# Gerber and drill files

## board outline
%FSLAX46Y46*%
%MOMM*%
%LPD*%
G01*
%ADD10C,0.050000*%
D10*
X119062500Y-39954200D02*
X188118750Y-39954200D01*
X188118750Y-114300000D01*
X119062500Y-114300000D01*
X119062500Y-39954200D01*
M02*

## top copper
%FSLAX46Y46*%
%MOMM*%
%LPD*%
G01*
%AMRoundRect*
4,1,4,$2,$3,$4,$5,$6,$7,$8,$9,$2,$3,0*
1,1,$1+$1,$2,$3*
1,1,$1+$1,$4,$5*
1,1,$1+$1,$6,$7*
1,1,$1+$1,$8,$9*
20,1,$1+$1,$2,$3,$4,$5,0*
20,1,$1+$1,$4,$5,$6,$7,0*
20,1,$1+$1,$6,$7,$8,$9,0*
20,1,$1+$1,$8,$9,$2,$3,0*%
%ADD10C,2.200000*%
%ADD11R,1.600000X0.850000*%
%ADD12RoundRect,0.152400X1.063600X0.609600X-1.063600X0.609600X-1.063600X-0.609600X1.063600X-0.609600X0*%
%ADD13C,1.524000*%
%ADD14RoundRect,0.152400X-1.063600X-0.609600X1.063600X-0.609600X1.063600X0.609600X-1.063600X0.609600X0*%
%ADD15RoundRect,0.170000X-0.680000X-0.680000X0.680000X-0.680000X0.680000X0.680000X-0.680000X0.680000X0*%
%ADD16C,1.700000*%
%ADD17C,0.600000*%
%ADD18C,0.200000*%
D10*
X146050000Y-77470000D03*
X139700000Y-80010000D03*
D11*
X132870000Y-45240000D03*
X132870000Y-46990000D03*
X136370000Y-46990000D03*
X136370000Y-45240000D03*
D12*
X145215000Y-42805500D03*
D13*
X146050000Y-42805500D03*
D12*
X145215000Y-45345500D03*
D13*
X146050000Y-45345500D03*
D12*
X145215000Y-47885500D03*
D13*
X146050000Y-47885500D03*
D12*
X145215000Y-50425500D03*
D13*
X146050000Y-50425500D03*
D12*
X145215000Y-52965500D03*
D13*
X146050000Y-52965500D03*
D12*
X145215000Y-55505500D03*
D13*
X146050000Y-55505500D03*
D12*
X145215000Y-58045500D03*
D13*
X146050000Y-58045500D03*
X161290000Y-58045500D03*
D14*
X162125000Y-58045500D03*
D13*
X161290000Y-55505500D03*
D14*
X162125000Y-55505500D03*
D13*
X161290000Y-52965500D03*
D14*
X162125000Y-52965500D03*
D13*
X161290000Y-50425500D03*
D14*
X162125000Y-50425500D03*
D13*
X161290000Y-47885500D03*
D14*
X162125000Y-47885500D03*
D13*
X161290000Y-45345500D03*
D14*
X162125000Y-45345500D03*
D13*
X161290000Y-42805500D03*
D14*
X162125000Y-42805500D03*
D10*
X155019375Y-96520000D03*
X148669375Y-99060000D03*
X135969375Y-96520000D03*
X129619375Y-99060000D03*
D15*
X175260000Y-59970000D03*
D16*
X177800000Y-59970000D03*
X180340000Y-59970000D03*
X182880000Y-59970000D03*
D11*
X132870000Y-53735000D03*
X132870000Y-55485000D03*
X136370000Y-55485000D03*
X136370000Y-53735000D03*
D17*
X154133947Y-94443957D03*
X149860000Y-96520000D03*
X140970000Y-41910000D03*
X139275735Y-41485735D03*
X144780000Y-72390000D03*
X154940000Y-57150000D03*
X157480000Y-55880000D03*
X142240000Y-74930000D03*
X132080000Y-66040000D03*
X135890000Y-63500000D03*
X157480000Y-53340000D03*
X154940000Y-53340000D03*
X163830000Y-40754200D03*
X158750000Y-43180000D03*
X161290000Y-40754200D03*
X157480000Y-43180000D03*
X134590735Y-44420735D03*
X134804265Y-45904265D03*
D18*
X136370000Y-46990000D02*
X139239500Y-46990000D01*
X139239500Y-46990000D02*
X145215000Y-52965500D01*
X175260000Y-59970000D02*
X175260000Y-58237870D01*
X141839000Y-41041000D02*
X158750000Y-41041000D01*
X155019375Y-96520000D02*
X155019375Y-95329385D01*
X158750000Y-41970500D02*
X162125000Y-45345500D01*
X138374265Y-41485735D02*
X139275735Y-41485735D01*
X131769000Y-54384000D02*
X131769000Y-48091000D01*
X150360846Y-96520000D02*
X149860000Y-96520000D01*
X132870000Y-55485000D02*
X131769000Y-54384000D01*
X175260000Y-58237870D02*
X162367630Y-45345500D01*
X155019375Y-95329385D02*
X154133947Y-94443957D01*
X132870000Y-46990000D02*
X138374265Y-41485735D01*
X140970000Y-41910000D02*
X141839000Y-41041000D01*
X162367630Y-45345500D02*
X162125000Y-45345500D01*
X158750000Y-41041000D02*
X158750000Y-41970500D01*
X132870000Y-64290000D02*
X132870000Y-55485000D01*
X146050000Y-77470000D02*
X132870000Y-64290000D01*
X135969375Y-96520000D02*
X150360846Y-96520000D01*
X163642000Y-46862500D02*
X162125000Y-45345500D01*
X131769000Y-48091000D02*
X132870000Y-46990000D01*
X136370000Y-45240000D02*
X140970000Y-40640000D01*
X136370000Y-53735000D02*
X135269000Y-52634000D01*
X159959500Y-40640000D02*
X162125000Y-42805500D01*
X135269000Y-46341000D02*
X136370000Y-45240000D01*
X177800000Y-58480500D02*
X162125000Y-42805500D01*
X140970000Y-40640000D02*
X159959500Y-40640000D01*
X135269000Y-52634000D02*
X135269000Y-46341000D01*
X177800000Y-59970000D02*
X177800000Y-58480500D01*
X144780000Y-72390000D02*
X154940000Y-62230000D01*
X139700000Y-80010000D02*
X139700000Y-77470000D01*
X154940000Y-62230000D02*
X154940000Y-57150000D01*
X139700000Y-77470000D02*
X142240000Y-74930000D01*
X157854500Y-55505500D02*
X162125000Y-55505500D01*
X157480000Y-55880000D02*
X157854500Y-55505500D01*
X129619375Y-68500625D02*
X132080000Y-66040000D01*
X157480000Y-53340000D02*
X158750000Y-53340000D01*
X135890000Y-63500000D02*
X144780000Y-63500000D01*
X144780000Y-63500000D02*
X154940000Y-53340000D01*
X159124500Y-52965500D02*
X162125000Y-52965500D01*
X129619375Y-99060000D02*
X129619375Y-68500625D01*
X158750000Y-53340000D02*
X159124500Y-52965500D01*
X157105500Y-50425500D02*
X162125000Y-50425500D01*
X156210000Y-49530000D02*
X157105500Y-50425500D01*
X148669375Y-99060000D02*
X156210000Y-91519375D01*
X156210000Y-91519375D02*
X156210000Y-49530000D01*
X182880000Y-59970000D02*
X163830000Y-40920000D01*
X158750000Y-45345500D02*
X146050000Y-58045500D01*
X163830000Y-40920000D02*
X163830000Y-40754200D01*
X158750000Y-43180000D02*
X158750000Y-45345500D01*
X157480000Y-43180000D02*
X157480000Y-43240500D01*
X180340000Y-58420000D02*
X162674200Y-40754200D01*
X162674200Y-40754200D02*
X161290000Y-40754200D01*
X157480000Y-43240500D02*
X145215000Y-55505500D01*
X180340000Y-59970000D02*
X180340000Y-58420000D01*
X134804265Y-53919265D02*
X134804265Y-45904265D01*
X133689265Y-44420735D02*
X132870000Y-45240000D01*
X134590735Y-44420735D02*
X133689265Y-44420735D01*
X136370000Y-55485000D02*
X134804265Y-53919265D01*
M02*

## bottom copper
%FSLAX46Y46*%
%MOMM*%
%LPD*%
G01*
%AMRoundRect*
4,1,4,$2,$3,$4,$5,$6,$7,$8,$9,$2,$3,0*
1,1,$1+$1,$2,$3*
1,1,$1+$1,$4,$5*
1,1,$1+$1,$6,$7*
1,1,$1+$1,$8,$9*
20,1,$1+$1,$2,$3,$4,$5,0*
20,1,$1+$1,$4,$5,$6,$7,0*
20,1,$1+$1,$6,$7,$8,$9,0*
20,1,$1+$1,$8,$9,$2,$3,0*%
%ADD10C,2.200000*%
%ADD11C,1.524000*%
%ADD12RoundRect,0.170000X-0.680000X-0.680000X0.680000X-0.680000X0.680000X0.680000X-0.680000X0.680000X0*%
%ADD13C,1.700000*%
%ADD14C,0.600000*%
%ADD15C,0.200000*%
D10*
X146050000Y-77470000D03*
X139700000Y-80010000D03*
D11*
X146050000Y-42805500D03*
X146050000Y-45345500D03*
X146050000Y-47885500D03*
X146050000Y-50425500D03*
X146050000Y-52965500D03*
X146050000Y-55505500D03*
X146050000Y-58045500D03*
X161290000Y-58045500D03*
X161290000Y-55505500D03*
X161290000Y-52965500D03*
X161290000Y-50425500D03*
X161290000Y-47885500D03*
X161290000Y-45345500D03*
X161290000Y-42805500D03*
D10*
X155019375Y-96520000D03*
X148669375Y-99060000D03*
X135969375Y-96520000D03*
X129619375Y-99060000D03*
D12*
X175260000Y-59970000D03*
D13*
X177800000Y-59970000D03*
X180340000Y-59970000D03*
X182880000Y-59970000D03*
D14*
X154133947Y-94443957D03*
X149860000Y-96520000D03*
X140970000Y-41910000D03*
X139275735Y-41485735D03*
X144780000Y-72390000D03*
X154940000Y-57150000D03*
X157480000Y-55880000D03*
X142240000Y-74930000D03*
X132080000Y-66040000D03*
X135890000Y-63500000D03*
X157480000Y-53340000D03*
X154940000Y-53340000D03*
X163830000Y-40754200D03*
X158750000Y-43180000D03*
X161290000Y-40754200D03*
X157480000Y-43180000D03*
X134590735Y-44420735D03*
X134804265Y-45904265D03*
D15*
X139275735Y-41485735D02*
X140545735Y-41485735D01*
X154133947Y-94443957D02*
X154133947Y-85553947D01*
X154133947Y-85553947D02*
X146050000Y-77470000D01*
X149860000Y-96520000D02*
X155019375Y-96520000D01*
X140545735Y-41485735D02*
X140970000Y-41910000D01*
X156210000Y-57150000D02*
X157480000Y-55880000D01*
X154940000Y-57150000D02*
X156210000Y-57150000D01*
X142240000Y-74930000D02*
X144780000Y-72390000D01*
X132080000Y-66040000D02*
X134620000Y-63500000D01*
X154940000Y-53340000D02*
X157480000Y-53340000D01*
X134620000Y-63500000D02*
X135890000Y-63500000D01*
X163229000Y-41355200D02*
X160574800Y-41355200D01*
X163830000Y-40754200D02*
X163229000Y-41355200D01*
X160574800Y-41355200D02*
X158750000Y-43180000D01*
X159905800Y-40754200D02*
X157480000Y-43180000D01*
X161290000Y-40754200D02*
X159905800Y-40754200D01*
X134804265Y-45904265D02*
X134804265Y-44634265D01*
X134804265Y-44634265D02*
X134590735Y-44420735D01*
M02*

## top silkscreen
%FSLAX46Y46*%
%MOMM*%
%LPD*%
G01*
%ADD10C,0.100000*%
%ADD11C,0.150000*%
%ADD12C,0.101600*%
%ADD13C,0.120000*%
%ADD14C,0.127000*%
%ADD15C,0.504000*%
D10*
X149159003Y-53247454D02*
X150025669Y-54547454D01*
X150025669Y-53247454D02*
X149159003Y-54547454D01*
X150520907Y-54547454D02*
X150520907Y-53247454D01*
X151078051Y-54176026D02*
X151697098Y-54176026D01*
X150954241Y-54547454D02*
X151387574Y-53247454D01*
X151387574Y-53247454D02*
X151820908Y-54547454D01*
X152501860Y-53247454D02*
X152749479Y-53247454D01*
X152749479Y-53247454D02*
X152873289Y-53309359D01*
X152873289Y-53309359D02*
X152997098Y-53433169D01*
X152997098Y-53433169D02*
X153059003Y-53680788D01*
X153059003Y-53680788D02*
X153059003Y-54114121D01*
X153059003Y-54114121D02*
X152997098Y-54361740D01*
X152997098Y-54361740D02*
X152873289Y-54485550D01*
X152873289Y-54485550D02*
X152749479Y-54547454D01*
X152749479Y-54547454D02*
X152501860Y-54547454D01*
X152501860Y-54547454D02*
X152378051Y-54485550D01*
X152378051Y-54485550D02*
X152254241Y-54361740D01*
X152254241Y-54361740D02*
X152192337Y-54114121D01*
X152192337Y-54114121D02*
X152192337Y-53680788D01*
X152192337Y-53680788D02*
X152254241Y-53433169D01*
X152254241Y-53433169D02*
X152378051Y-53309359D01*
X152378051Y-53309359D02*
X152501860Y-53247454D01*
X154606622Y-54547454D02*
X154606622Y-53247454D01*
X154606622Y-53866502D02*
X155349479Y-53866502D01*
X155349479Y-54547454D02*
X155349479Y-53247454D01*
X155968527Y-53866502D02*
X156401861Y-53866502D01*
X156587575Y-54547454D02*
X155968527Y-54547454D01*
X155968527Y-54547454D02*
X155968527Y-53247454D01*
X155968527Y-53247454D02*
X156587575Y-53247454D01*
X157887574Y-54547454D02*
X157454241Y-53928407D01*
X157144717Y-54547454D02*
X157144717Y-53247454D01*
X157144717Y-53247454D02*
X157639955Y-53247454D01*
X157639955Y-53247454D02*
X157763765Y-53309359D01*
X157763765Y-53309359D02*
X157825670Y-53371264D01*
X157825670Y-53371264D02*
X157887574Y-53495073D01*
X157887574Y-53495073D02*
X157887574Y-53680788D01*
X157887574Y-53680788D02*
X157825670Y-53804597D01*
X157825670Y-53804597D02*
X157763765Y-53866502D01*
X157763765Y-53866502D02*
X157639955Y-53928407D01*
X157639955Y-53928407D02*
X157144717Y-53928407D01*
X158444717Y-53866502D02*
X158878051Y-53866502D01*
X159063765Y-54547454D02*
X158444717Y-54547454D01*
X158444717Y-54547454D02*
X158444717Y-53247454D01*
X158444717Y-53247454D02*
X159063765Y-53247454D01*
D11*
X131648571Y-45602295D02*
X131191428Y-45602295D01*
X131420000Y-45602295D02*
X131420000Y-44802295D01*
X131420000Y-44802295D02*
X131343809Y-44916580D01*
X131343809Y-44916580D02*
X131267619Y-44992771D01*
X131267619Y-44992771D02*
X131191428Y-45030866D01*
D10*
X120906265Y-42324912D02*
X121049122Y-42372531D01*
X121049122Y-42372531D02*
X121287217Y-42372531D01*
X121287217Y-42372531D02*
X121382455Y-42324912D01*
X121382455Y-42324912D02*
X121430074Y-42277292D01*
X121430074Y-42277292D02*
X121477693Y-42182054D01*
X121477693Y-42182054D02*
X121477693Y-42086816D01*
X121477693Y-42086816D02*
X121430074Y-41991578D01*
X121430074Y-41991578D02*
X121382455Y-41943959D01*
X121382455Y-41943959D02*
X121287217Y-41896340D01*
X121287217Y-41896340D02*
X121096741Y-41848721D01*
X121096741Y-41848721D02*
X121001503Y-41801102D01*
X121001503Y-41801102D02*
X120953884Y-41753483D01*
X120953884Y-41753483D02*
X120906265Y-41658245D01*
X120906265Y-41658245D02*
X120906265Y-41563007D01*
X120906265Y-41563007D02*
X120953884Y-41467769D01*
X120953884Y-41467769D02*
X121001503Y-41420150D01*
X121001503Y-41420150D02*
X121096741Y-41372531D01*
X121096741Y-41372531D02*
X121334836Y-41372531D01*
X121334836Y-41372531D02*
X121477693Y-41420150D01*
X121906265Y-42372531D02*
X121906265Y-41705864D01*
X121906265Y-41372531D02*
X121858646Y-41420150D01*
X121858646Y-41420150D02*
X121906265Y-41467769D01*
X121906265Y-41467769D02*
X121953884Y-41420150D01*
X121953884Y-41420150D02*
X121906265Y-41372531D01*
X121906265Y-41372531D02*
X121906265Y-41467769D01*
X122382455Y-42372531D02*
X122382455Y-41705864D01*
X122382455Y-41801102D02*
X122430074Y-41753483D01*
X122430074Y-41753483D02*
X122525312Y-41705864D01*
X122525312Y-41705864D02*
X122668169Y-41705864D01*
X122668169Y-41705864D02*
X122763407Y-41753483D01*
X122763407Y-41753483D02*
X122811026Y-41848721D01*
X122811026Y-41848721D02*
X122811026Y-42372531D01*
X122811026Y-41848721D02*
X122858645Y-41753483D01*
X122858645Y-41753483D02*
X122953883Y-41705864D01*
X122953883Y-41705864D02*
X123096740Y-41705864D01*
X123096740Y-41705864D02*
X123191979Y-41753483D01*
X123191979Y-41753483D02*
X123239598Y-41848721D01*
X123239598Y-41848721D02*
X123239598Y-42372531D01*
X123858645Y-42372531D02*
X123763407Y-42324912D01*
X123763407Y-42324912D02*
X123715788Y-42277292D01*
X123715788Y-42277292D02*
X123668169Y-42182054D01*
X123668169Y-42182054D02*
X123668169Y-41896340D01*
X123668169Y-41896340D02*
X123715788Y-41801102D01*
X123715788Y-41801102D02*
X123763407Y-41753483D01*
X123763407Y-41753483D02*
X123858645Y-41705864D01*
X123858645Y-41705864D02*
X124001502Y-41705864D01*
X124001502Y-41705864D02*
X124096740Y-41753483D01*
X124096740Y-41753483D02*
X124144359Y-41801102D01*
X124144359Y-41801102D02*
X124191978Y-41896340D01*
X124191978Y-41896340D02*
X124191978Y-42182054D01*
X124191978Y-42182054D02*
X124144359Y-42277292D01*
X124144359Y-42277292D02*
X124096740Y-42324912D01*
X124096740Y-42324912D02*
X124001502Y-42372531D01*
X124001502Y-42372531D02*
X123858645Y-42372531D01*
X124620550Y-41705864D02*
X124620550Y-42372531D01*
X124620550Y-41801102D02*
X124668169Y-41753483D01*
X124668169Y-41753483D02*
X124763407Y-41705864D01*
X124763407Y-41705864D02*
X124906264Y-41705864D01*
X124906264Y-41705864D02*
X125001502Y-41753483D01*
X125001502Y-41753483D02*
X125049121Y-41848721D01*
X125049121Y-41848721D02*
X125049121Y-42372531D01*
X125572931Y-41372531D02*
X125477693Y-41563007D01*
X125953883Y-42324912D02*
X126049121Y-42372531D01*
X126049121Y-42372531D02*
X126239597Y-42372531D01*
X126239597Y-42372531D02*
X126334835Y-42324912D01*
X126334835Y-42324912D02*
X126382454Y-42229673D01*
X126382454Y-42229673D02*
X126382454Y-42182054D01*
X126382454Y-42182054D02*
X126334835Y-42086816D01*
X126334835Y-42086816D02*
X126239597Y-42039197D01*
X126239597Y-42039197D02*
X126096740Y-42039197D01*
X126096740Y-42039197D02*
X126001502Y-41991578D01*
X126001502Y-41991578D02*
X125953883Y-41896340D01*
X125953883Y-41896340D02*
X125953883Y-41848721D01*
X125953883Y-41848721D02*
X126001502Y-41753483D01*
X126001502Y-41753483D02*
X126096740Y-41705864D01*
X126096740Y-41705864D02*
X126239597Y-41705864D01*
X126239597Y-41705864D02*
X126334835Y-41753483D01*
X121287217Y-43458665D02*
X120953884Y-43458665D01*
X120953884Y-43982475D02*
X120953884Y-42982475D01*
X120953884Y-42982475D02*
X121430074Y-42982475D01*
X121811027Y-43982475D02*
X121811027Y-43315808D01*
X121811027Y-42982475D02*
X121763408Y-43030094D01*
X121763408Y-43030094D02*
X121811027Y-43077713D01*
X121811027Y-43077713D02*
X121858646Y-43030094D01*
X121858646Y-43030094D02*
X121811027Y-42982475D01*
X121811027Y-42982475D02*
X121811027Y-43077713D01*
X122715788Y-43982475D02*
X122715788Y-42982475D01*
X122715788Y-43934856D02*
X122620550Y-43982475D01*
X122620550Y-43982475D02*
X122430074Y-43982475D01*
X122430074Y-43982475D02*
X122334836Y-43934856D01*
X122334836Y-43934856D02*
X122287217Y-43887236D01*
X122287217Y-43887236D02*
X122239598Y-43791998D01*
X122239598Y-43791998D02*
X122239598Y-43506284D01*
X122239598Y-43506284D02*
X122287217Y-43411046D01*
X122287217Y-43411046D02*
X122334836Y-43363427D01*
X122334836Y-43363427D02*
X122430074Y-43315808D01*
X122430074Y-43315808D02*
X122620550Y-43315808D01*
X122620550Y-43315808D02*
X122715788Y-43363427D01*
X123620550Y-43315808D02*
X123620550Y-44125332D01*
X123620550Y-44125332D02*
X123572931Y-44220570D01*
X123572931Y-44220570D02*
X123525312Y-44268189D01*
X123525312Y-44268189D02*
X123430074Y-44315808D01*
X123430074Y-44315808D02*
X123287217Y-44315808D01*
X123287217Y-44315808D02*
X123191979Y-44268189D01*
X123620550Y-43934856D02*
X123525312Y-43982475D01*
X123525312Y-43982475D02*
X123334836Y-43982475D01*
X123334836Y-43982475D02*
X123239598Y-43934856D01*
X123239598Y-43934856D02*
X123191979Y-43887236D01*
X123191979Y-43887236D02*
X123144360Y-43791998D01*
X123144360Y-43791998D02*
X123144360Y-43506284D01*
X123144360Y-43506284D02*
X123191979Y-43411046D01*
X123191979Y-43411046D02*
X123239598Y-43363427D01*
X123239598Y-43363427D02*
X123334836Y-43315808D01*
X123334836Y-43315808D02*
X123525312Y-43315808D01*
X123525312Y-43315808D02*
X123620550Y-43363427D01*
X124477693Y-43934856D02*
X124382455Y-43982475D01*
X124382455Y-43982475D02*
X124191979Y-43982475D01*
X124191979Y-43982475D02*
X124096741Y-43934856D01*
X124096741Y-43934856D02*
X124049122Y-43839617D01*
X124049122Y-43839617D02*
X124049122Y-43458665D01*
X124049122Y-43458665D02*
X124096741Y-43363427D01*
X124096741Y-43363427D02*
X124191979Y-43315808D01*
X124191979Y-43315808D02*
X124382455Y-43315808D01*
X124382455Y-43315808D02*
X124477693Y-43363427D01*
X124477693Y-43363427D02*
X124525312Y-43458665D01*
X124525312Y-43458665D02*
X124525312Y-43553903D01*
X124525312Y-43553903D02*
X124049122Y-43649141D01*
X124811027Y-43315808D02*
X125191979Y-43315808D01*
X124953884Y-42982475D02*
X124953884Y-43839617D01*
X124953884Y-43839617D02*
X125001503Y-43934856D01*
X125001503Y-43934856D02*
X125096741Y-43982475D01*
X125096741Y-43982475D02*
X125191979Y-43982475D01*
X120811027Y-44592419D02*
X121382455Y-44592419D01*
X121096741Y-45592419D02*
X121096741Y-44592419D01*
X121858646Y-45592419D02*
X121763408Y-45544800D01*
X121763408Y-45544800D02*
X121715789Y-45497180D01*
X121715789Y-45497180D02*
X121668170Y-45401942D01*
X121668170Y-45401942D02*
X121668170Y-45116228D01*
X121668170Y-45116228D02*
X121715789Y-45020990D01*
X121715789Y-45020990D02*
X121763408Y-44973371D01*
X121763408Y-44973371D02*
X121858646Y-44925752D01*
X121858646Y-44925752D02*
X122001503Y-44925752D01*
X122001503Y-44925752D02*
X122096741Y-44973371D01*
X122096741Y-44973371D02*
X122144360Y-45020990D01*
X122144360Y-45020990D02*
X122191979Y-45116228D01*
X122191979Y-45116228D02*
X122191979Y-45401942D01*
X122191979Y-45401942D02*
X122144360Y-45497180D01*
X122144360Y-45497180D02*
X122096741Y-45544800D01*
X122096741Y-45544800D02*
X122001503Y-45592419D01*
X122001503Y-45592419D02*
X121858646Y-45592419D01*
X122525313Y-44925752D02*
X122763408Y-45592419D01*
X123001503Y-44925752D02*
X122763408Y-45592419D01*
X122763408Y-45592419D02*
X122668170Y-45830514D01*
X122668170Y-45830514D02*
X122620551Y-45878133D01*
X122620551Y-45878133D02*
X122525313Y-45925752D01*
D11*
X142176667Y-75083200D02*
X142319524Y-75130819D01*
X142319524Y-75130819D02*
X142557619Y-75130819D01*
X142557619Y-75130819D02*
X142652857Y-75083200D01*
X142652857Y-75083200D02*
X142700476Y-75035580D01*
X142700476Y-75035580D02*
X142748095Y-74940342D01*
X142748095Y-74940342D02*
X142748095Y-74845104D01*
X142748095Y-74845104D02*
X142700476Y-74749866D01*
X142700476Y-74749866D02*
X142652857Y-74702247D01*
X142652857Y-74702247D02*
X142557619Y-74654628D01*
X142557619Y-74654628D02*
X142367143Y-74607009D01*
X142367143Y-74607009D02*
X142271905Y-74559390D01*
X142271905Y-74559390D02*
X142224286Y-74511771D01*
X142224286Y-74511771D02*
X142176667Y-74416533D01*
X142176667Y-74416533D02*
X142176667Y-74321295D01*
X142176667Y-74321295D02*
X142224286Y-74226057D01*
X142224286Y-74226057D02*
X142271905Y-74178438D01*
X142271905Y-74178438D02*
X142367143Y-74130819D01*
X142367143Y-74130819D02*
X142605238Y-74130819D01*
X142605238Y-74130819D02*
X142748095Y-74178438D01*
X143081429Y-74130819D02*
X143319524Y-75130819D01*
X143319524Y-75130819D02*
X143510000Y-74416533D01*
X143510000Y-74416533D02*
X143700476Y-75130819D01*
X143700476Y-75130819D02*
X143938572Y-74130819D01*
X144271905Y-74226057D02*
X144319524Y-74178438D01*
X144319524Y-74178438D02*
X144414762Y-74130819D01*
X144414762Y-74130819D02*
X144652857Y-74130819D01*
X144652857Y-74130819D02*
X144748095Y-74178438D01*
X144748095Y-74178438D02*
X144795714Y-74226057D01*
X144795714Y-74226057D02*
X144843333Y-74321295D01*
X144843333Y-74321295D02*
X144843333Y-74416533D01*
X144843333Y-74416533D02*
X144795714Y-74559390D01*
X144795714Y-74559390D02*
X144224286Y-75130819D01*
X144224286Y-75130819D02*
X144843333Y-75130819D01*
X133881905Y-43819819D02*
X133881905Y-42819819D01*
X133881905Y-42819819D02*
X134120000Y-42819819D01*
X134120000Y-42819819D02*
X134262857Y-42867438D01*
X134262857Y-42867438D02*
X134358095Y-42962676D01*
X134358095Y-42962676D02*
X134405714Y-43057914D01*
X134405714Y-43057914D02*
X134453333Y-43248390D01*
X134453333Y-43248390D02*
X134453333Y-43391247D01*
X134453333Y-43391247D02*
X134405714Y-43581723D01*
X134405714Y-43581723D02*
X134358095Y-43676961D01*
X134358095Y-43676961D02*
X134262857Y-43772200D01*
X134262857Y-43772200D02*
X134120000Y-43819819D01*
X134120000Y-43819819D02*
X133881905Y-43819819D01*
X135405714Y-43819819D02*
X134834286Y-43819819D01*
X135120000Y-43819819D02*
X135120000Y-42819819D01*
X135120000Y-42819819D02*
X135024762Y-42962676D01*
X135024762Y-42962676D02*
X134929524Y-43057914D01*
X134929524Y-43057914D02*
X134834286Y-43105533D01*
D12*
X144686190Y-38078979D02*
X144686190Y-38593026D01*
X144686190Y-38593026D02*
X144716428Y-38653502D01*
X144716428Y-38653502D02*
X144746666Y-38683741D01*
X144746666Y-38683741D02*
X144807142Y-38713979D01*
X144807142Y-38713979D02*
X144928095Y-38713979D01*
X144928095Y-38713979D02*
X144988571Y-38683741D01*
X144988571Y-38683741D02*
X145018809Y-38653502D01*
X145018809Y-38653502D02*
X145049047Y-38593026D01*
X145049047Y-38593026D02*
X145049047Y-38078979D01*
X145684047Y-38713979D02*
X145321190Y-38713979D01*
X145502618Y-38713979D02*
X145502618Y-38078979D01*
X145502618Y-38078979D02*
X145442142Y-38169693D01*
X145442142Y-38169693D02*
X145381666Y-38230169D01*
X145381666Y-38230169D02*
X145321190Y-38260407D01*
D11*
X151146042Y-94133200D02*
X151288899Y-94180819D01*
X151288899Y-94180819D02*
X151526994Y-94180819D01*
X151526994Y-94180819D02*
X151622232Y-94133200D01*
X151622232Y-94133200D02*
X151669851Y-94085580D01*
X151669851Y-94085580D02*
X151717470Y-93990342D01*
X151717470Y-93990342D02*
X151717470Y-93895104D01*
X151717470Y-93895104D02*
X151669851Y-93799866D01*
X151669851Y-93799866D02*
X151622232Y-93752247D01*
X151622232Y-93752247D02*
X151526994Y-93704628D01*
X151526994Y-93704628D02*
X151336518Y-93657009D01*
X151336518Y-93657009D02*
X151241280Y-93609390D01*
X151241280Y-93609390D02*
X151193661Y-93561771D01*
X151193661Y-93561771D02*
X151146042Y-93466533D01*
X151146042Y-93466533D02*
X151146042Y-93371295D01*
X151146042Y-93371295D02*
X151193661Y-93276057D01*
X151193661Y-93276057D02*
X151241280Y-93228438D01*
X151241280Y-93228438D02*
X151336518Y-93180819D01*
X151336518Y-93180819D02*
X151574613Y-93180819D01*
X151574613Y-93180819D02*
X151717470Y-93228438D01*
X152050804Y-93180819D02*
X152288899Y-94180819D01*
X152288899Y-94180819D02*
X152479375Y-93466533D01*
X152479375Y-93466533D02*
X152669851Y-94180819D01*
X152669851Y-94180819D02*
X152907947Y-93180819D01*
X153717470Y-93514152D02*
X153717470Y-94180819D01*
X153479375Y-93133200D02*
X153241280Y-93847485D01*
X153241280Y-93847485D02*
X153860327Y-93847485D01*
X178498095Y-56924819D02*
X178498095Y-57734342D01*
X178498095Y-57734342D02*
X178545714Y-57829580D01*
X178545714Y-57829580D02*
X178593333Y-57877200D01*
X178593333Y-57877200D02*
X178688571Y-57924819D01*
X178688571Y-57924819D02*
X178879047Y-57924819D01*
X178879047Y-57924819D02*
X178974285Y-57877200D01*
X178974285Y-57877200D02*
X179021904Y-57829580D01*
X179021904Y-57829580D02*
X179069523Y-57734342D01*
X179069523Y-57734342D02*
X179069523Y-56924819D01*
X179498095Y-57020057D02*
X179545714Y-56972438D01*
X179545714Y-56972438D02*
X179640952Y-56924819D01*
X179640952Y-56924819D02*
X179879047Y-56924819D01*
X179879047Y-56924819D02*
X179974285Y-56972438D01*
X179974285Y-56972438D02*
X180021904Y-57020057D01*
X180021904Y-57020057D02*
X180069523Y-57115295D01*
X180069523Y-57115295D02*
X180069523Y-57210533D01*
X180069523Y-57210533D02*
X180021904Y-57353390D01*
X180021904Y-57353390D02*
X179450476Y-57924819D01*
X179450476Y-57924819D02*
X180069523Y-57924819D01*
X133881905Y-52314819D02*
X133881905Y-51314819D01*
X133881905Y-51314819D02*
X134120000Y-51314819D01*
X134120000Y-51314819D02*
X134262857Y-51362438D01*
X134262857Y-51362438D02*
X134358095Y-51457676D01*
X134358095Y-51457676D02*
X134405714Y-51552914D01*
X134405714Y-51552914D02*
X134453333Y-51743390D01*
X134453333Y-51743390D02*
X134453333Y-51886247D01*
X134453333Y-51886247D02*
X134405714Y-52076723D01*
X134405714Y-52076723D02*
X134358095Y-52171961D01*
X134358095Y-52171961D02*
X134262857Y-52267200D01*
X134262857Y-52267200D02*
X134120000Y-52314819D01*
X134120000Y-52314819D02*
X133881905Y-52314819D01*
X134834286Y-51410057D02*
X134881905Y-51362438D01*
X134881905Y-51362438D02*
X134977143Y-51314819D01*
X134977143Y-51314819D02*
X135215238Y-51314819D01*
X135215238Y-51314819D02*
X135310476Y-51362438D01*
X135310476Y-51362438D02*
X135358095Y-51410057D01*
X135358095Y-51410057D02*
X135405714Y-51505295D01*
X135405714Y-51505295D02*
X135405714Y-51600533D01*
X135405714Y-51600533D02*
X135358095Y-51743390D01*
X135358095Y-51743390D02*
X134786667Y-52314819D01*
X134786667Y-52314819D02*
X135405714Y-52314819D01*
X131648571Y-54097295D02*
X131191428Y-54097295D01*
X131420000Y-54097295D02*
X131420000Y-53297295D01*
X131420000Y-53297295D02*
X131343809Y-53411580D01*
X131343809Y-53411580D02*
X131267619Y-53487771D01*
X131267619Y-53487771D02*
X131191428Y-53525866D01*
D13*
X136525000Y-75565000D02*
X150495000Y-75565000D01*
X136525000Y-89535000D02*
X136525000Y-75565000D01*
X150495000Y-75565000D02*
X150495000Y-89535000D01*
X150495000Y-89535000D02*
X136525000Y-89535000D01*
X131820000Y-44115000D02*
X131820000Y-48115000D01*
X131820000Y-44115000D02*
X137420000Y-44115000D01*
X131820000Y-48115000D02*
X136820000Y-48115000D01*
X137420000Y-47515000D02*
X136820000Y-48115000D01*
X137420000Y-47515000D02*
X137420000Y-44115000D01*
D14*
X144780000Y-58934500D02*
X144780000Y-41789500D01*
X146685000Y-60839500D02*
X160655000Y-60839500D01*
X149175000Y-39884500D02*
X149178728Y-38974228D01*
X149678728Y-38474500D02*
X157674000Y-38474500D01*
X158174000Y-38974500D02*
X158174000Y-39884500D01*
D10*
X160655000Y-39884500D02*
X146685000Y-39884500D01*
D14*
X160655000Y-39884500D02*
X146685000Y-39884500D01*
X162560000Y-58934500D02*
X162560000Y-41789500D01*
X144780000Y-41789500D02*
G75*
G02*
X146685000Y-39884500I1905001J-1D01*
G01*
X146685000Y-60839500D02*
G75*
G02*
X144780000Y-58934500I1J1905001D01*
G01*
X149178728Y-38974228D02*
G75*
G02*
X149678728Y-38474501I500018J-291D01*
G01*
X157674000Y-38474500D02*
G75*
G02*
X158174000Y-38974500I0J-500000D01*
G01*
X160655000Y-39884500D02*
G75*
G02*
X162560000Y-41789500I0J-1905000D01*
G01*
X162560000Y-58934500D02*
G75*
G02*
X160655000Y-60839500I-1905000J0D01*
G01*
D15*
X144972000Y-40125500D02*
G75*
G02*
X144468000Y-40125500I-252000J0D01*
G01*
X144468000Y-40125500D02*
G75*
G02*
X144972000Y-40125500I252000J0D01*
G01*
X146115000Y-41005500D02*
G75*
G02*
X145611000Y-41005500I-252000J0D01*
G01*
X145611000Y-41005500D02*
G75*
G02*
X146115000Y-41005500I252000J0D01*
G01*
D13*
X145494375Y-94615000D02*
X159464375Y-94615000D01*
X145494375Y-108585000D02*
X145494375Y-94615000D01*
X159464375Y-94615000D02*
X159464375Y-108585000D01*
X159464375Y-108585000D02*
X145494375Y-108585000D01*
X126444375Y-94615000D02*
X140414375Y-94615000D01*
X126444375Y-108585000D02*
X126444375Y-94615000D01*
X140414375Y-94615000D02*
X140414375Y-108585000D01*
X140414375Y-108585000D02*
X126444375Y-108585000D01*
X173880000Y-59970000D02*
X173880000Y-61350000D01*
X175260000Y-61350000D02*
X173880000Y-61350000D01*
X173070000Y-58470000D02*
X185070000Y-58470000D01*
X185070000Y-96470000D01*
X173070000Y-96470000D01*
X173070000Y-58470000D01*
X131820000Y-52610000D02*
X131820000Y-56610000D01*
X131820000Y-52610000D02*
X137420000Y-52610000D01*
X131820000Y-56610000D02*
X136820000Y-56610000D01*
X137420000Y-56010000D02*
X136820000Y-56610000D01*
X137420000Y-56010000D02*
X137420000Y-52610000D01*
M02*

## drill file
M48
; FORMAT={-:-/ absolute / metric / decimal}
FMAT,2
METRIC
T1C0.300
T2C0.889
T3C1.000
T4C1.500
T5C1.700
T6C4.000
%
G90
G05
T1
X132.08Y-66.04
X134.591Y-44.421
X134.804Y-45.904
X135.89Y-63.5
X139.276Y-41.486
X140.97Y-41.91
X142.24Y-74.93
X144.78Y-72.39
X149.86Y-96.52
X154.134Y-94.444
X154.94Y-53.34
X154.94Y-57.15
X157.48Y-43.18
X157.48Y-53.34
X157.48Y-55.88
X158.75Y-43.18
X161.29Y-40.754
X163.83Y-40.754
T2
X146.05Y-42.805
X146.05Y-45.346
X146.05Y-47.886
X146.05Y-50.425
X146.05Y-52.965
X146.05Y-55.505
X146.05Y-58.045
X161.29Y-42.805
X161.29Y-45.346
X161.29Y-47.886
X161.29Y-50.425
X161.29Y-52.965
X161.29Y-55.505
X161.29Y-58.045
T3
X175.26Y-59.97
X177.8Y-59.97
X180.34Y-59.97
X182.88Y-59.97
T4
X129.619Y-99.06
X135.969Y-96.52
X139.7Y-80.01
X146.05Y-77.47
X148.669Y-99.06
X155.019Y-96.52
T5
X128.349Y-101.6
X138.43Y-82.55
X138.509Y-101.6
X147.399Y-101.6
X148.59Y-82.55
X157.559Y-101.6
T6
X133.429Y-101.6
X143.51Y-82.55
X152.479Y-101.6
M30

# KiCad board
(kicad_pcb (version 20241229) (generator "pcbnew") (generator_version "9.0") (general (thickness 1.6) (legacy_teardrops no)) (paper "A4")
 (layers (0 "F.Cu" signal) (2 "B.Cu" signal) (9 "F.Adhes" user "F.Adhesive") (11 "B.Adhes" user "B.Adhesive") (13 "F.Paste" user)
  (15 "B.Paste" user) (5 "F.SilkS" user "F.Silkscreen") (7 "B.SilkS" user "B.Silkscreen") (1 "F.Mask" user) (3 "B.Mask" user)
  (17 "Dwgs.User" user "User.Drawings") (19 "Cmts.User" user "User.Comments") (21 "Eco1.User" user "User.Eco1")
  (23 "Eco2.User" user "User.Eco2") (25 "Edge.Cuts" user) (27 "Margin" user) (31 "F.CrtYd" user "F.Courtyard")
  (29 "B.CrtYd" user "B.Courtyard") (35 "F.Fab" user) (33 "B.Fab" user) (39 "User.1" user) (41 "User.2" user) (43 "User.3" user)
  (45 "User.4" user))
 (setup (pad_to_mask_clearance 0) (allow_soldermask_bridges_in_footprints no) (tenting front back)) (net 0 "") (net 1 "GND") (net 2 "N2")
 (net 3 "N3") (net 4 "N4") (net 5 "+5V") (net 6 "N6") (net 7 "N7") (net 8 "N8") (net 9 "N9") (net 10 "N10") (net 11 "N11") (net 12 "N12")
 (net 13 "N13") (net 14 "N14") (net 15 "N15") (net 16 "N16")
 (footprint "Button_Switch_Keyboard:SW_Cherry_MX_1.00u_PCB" (layer "F.Cu") (at 146.05 77.47)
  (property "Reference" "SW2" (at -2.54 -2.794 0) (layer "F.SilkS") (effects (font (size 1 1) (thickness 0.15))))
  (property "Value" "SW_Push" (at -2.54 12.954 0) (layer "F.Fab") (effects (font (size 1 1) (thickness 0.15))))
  (fp_line (start -9.525 -1.905) (end 4.445 -1.905) (stroke (width 0.12) (type solid)) (layer "F.SilkS"))
  (fp_line (start -9.525 12.065) (end -9.525 -1.905) (stroke (width 0.12) (type solid)) (layer "F.SilkS"))
  (fp_line (start 4.445 -1.905) (end 4.445 12.065) (stroke (width 0.12) (type solid)) (layer "F.SilkS"))
  (fp_line (start 4.445 12.065) (end -9.525 12.065) (stroke (width 0.12) (type solid)) (layer "F.SilkS"))
  (pad "" np_thru_hole circle (at -7.62 5.08) (size 1.7 1.7) (drill 1.7) (layers "*.Cu" "*.Mask"))
  (pad "" np_thru_hole circle (at -2.54 5.08) (size 4 4) (drill 4) (layers "*.Cu" "*.Mask"))
  (pad "" np_thru_hole circle (at 2.54 5.08) (size 1.7 1.7) (drill 1.7) (layers "*.Cu" "*.Mask"))
  (pad "1" thru_hole circle (at 0 0) (size 2.2 2.2) (drill 1.5) (layers "*.Cu" "*.Mask") (remove_unused_layers no) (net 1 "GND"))
  (pad "2" thru_hole circle (at -6.35 2.54) (size 2.2 2.2) (drill 1.5) (layers "*.Cu" "*.Mask") (remove_unused_layers no) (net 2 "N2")))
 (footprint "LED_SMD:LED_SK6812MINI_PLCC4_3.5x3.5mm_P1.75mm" (layer "F.Cu") (at 134.62 46.115)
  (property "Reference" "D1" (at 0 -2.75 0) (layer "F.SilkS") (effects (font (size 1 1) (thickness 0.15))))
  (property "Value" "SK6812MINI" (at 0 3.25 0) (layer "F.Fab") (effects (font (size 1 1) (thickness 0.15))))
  (fp_line (start -2.8 -2) (end -2.8 2) (stroke (width 0.12) (type default)) (layer "F.SilkS"))
  (fp_line (start -2.8 -2) (end 2.8 -2) (stroke (width 0.12) (type solid)) (layer "F.SilkS"))
  (fp_line (start -2.8 2) (end 2.2 2) (stroke (width 0.12) (type solid)) (layer "F.SilkS"))
  (fp_line (start 2.8 1.4) (end 2.2 2) (stroke (width 0.12) (type default)) (layer "F.SilkS"))
  (fp_line (start 2.8 1.4) (end 2.8 -2) (stroke (width 0.12) (type solid)) (layer "F.SilkS"))
  (pad "1" smd rect (at -1.75 -0.875) (size 1.6 0.85) (layers "F.Cu" "F.Mask" "F.Paste") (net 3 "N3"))
  (pad "2" smd rect (at -1.75 0.875) (size 1.6 0.85) (layers "F.Cu" "F.Mask" "F.Paste") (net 1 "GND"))
  (pad "3" smd rect (at 1.75 0.875) (size 1.6 0.85) (layers "F.Cu" "F.Mask" "F.Paste") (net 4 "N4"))
  (pad "4" smd rect (at 1.75 -0.875) (size 1.6 0.85) (layers "F.Cu" "F.Mask" "F.Paste") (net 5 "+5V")))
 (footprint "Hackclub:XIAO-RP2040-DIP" (layer "F.Cu") (at 153.67 50.4255)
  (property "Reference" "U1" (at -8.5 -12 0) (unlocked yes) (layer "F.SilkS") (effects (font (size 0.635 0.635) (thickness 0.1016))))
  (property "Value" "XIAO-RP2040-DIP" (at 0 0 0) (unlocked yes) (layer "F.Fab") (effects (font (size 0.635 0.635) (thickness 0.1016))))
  (fp_line (start -8.89 8.509) (end -8.89 -8.636) (stroke (width 0.127) (type solid)) (layer "F.SilkS"))
  (fp_line (start -6.985 10.414) (end 6.985 10.414) (stroke (width 0.127) (type solid)) (layer "F.SilkS"))
  (fp_line (start -4.495 -10.541) (end -4.491272 -11.451272) (stroke (width 0.127) (type solid)) (layer "F.SilkS"))
  (fp_line (start -3.991272 -11.951) (end 4.004 -11.951) (stroke (width 0.127) (type solid)) (layer "F.SilkS"))
  (fp_line (start 4.504 -11.451) (end 4.504 -10.541) (stroke (width 0.127) (type solid)) (layer "F.SilkS"))
  (fp_line (start 6.985 -10.541) (end -6.985 -10.541) (stroke (width 0.1) (type solid)) (layer "F.SilkS"))
  (fp_line (start 6.985 -10.541) (end -6.985 -10.541) (stroke (width 0.127) (type solid)) (layer "F.SilkS"))
  (fp_line (start 8.89 8.509) (end 8.89 -8.636) (stroke (width 0.127) (type solid)) (layer "F.SilkS"))
  (fp_arc (start -8.89 -8.636) (mid -8.332038 -9.983038) (end -6.985 -10.541) (stroke (width 0.127) (type solid)) (layer "F.SilkS"))
  (fp_arc (start -6.985 10.414) (mid -8.332038 9.856038) (end -8.89 8.509) (stroke (width 0.127) (type solid)) (layer "F.SilkS"))
  (fp_arc (start -4.491272 -11.451272) (mid -4.344728 -11.80464) (end -3.991272 -11.951) (stroke (width 0.127) (type default))
   (layer "F.SilkS"))
  (fp_arc (start 4.004 -11.951) (mid 4.357553 -11.804553) (end 4.504 -11.451) (stroke (width 0.127) (type default)) (layer "F.SilkS"))
  (fp_arc (start 6.985 -10.541) (mid 8.332038 -9.983038) (end 8.89 -8.636) (stroke (width 0.127) (type solid)) (layer "F.SilkS"))
  (fp_arc (start 8.89 8.509) (mid 8.332038 9.856038) (end 6.985 10.414) (stroke (width 0.127) (type solid)) (layer "F.SilkS"))
  (fp_circle (center -8.95 -10.3) (end -8.95 -10.554) (stroke (width 0.5) (type solid)) (fill yes) (layer "F.SilkS"))
  (fp_circle (center -7.807 -9.42) (end -7.807 -9.674) (stroke (width 0.5) (type solid)) (fill yes) (layer "F.SilkS"))
  (pad "1" smd roundrect (at -8.455 -7.62 180) (size 2.432 1.524) (layers "F.Cu" "F.Mask") (roundrect_rratio 0.1) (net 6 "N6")
   (thermal_bridge_angle 45))
  (pad "1" thru_hole circle (at -7.62 -7.62 180) (size 1.524 1.524) (drill 0.889) (layers "*.Cu" "*.Mask") (remove_unused_layers no)
   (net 6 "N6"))
  (pad "2" smd roundrect (at -8.455 -5.08 180) (size 2.432 1.524) (layers "F.Cu" "F.Mask") (roundrect_rratio 0.1) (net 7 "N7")
   (thermal_bridge_angle 45))
  (pad "2" thru_hole circle (at -7.62 -5.08 180) (size 1.524 1.524) (drill 0.889) (layers "*.Cu" "*.Mask") (remove_unused_layers no)
   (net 7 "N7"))
  (pad "3" smd roundrect (at -8.455 -2.54 180) (size 2.432 1.524) (layers "F.Cu" "F.Mask") (roundrect_rratio 0.1) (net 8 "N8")
   (thermal_bridge_angle 45))
  (pad "3" thru_hole circle (at -7.62 -2.54 180) (size 1.524 1.524) (drill 0.889) (layers "*.Cu" "*.Mask") (remove_unused_layers no)
   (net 8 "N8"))
  (pad "4" smd roundrect (at -8.455 0 180) (size 2.432 1.524) (layers "F.Cu" "F.Mask") (roundrect_rratio 0.1) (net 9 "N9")
   (thermal_bridge_angle 45))
  (pad "4" thru_hole circle (at -7.62 0 180) (size 1.524 1.524) (drill 0.889) (layers "*.Cu" "*.Mask") (remove_unused_layers no)
   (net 9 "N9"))
  (pad "5" smd roundrect (at -8.455 2.54 180) (size 2.432 1.524) (layers "F.Cu" "F.Mask") (roundrect_rratio 0.1) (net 4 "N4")
   (thermal_bridge_angle 45))
  (pad "5" thru_hole circle (at -7.62 2.54 180) (size 1.524 1.524) (drill 0.889) (layers "*.Cu" "*.Mask") (remove_unused_layers no)
   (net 4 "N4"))
  (pad "6" smd roundrect (at -8.455 5.08 180) (size 2.432 1.524) (layers "F.Cu" "F.Mask") (roundrect_rratio 0.1) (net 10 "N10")
   (thermal_bridge_angle 45))
  (pad "6" thru_hole circle (at -7.62 5.08 180) (size 1.524 1.524) (drill 0.889) (layers "*.Cu" "*.Mask") (remove_unused_layers no)
   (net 10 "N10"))
  (pad "7" smd roundrect (at -8.455 7.62 180) (size 2.432 1.524) (layers "F.Cu" "F.Mask") (roundrect_rratio 0.1) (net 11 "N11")
   (thermal_bridge_angle 45))
  (pad "7" thru_hole circle (at -7.62 7.62 180) (size 1.524 1.524) (drill 0.889) (layers "*.Cu" "*.Mask") (remove_unused_layers no)
   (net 11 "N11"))
  (pad "8" thru_hole circle (at 7.62 7.62) (size 1.524 1.524) (drill 0.889) (layers "*.Cu" "*.Mask") (remove_unused_layers no)
   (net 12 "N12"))
  (pad "8" smd roundrect (at 8.455 7.62) (size 2.432 1.524) (layers "F.Cu" "F.Mask") (roundrect_rratio 0.1) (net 12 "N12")
   (thermal_bridge_angle 45))
  (pad "9" thru_hole circle (at 7.62 5.08) (size 1.524 1.524) (drill 0.889) (layers "*.Cu" "*.Mask") (remove_unused_layers no) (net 2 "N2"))
  (pad "9" smd roundrect (at 8.455 5.08) (size 2.432 1.524) (layers "F.Cu" "F.Mask") (roundrect_rratio 0.1) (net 2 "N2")
   (thermal_bridge_angle 45))
  (pad "10" thru_hole circle (at 7.62 2.54) (size 1.524 1.524) (drill 0.889) (layers "*.Cu" "*.Mask") (remove_unused_layers no)
   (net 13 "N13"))
  (pad "10" smd roundrect (at 8.455 2.54) (size 2.432 1.524) (layers "F.Cu" "F.Mask") (roundrect_rratio 0.1) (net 13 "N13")
   (thermal_bridge_angle 45))
  (pad "11" thru_hole circle (at 7.62 0) (size 1.524 1.524) (drill 0.889) (layers "*.Cu" "*.Mask") (remove_unused_layers no) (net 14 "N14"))
  (pad "11" smd roundrect (at 8.455 0) (size 2.432 1.524) (layers "F.Cu" "F.Mask") (roundrect_rratio 0.1) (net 14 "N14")
   (thermal_bridge_angle 45))
  (pad "12" thru_hole circle (at 7.62 -2.54) (size 1.524 1.524) (drill 0.889) (layers "*.Cu" "*.Mask") (remove_unused_layers no)
   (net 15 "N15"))
  (pad "12" smd roundrect (at 8.455 -2.54) (size 2.432 1.524) (layers "F.Cu" "F.Mask") (roundrect_rratio 0.1) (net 15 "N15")
   (thermal_bridge_angle 45))
  (pad "13" thru_hole circle (at 7.62 -5.08) (size 1.524 1.524) (drill 0.889) (layers "*.Cu" "*.Mask") (remove_unused_layers no)
   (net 1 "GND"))
  (pad "13" smd roundrect (at 8.455 -5.08) (size 2.432 1.524) (layers "F.Cu" "F.Mask") (roundrect_rratio 0.1) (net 1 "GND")
   (thermal_bridge_angle 45))
  (pad "14" thru_hole circle (at 7.62 -7.62) (size 1.524 1.524) (drill 0.889) (layers "*.Cu" "*.Mask") (remove_unused_layers no)
   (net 5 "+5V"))
  (pad "14" smd roundrect (at 8.455 -7.62) (size 2.432 1.524) (layers "F.Cu" "F.Mask") (roundrect_rratio 0.1) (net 5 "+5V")
   (thermal_bridge_angle 45)))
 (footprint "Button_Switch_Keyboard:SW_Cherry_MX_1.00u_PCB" (layer "F.Cu") (at 155.019375 96.52)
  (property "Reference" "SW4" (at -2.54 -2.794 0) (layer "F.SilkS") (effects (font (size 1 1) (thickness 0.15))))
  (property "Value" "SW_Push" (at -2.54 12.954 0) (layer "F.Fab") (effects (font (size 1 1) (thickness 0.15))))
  (fp_line (start -9.525 -1.905) (end 4.445 -1.905) (stroke (width 0.12) (type solid)) (layer "F.SilkS"))
  (fp_line (start -9.525 12.065) (end -9.525 -1.905) (stroke (width 0.12) (type solid)) (layer "F.SilkS"))
  (fp_line (start 4.445 -1.905) (end 4.445 12.065) (stroke (width 0.12) (type solid)) (layer "F.SilkS"))
  (fp_line (start 4.445 12.065) (end -9.525 12.065) (stroke (width 0.12) (type solid)) (layer "F.SilkS"))
  (pad "" np_thru_hole circle (at -7.62 5.08) (size 1.7 1.7) (drill 1.7) (layers "*.Cu" "*.Mask"))
  (pad "" np_thru_hole circle (at -2.54 5.08) (size 4 4) (drill 4) (layers "*.Cu" "*.Mask"))
  (pad "" np_thru_hole circle (at 2.54 5.08) (size 1.7 1.7) (drill 1.7) (layers "*.Cu" "*.Mask"))
  (pad "1" thru_hole circle (at 0 0) (size 2.2 2.2) (drill 1.5) (layers "*.Cu" "*.Mask") (remove_unused_layers no) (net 1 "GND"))
  (pad "2" thru_hole circle (at -6.35 2.54) (size 2.2 2.2) (drill 1.5) (layers "*.Cu" "*.Mask") (remove_unused_layers no) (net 14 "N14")))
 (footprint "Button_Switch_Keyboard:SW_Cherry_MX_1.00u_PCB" (layer "F.Cu") (at 135.969375 96.52)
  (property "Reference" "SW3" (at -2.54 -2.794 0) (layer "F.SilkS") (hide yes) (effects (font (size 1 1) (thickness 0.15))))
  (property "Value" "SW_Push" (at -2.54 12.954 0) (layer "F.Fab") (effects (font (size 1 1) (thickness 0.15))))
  (fp_line (start -9.525 -1.905) (end 4.445 -1.905) (stroke (width 0.12) (type solid)) (layer "F.SilkS"))
  (fp_line (start -9.525 12.065) (end -9.525 -1.905) (stroke (width 0.12) (type solid)) (layer "F.SilkS"))
  (fp_line (start 4.445 -1.905) (end 4.445 12.065) (stroke (width 0.12) (type solid)) (layer "F.SilkS"))
  (fp_line (start 4.445 12.065) (end -9.525 12.065) (stroke (width 0.12) (type solid)) (layer "F.SilkS"))
  (pad "" np_thru_hole circle (at -7.62 5.08) (size 1.7 1.7) (drill 1.7) (layers "*.Cu" "*.Mask"))
  (pad "" np_thru_hole circle (at -2.54 5.08) (size 4 4) (drill 4) (layers "*.Cu" "*.Mask"))
  (pad "" np_thru_hole circle (at 2.54 5.08) (size 1.7 1.7) (drill 1.7) (layers "*.Cu" "*.Mask"))
  (pad "1" thru_hole circle (at 0 0) (size 2.2 2.2) (drill 1.5) (layers "*.Cu" "*.Mask") (remove_unused_layers no) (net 1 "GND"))
  (pad "2" thru_hole circle (at -6.35 2.54) (size 2.2 2.2) (drill 1.5) (layers "*.Cu" "*.Mask") (remove_unused_layers no) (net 13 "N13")))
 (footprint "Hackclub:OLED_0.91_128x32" (layer "F.Cu") (at 175.26 59.97)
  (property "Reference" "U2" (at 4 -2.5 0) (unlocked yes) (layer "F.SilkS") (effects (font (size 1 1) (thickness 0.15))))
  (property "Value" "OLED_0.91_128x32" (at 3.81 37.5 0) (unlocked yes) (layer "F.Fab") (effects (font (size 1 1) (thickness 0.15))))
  (fp_line (start -1.38 0) (end -1.38 1.38) (stroke (width 0.12) (type solid)) (layer "F.SilkS"))
  (fp_line (start 0 1.38) (end -1.38 1.38) (stroke (width 0.12) (type solid)) (layer "F.SilkS"))
  (fp_rect (start -2.19 -1.5) (end 9.81 36.5) (stroke (width 0.12) (type solid)) (fill no) (layer "F.SilkS"))
  (pad "1" thru_hole roundrect (at 0 0) (size 1.7 1.7) (drill 1) (layers "*.Cu" "*.Mask") (remove_unused_layers no) (roundrect_rratio 0.1)
   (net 1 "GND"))
  (pad "2" thru_hole circle (at 2.54 0) (size 1.7 1.7) (drill 1) (layers "*.Cu" "*.Mask") (remove_unused_layers no) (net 5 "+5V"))
  (pad "3" thru_hole circle (at 5.08 0) (size 1.7 1.7) (drill 1) (layers "*.Cu" "*.Mask") (remove_unused_layers no) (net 10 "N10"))
  (pad "4" thru_hole circle (at 7.62 0) (size 1.7 1.7) (drill 1) (layers "*.Cu" "*.Mask") (remove_unused_layers no) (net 11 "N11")))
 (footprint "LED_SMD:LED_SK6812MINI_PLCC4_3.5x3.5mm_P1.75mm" (layer "F.Cu") (at 134.62 54.61)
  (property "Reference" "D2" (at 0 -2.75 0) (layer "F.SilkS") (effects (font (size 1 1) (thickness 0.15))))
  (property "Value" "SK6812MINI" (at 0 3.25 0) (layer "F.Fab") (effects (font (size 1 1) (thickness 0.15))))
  (fp_line (start -2.8 -2) (end -2.8 2) (stroke (width 0.12) (type default)) (layer "F.SilkS"))
  (fp_line (start -2.8 -2) (end 2.8 -2) (stroke (width 0.12) (type solid)) (layer "F.SilkS"))
  (fp_line (start -2.8 2) (end 2.2 2) (stroke (width 0.12) (type solid)) (layer "F.SilkS"))
  (fp_line (start 2.8 1.4) (end 2.2 2) (stroke (width 0.12) (type default)) (layer "F.SilkS"))
  (fp_line (start 2.8 1.4) (end 2.8 -2) (stroke (width 0.12) (type solid)) (layer "F.SilkS"))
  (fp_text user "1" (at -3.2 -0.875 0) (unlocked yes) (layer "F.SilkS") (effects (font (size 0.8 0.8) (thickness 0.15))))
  (pad "1" smd rect (at -1.75 -0.875) (size 1.6 0.85) (layers "F.Cu" "F.Mask" "F.Paste") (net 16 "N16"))
  (pad "2" smd rect (at -1.75 0.875) (size 1.6 0.85) (layers "F.Cu" "F.Mask" "F.Paste") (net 1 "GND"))
  (pad "3" smd rect (at 1.75 0.875) (size 1.6 0.85) (layers "F.Cu" "F.Mask" "F.Paste") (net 3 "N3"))
  (pad "4" smd rect (at 1.75 -0.875) (size 1.6 0.85) (layers "F.Cu" "F.Mask" "F.Paste") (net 5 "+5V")))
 (gr_rect (start 119.0625 39.9542) (end 188.11875 114.3) (stroke (width 0.05) (type default)) (fill no) (layer "Edge.Cuts"))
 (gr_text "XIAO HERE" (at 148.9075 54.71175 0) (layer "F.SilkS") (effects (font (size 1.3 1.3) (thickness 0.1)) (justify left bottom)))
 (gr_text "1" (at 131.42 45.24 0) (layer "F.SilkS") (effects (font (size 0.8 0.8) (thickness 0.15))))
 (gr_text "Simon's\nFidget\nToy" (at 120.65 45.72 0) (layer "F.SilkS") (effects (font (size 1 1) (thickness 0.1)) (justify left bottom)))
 (segment (start 136.37 46.99) (end 139.2395 46.99) (width 0.2) (layer "F.Cu") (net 4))
 (segment (start 139.2395 46.99) (end 145.215 52.9655) (width 0.2) (layer "F.Cu") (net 4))
 (segment (start 175.26 59.97) (end 175.26 58.23787) (width 0.2) (layer "F.Cu") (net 1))
 (segment (start 141.839 41.041) (end 158.75 41.041) (width 0.2) (layer "F.Cu") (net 1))
 (segment (start 155.019375 96.52) (end 155.019375 95.329385) (width 0.2) (layer "F.Cu") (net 1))
 (segment (start 158.75 41.9705) (end 162.125 45.3455) (width 0.2) (layer "F.Cu") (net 1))
 (segment (start 138.374265 41.485735) (end 139.275735 41.485735) (width 0.2) (layer "F.Cu") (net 1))
 (segment (start 131.769 54.384) (end 131.769 48.091) (width 0.2) (layer "F.Cu") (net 1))
 (segment (start 150.360846 96.52) (end 149.86 96.52) (width 0.2) (layer "F.Cu") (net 1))
 (segment (start 132.87 55.485) (end 131.769 54.384) (width 0.2) (layer "F.Cu") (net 1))
 (segment (start 175.26 58.23787) (end 162.36763 45.3455) (width 0.2) (layer "F.Cu") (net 1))
 (segment (start 155.019375 95.329385) (end 154.133947 94.443957) (width 0.2) (layer "F.Cu") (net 1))
 (segment (start 132.87 46.99) (end 138.374265 41.485735) (width 0.2) (layer "F.Cu") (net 1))
 (segment (start 140.97 41.91) (end 141.839 41.041) (width 0.2) (layer "F.Cu") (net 1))
 (segment (start 162.36763 45.3455) (end 162.125 45.3455) (width 0.2) (layer "F.Cu") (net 1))
 (segment (start 158.75 41.041) (end 158.75 41.9705) (width 0.2) (layer "F.Cu") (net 1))
 (segment (start 132.87 64.29) (end 132.87 55.485) (width 0.2) (layer "F.Cu") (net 1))
 (segment (start 146.05 77.47) (end 132.87 64.29) (width 0.2) (layer "F.Cu") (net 1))
 (segment (start 135.969375 96.52) (end 150.360846 96.52) (width 0.2) (layer "F.Cu") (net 1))
 (segment (start 163.642 46.8625) (end 162.125 45.3455) (width 0.2) (layer "F.Cu") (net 1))
 (segment (start 131.769 48.091) (end 132.87 46.99) (width 0.2) (layer "F.Cu") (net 1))
 (via (at 154.133947 94.443957) (size 0.6) (drill 0.3) (layers "F.Cu" "B.Cu") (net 1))
 (via (at 149.86 96.52) (size 0.6) (drill 0.3) (layers "F.Cu" "B.Cu") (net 1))
 (via (at 140.97 41.91) (size 0.6) (drill 0.3) (layers "F.Cu" "B.Cu") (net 1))
 (via (at 139.275735 41.485735) (size 0.6) (drill 0.3) (layers "F.Cu" "B.Cu") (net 1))
 (segment (start 139.275735 41.485735) (end 140.545735 41.485735) (width 0.2) (layer "B.Cu") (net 1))
 (segment (start 154.133947 94.443957) (end 154.133947 85.553947) (width 0.2) (layer "B.Cu") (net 1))
 (segment (start 154.133947 85.553947) (end 146.05 77.47) (width 0.2) (layer "B.Cu") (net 1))
 (segment (start 149.86 96.52) (end 155.019375 96.52) (width 0.2) (layer "B.Cu") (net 1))
 (segment (start 140.545735 41.485735) (end 140.97 41.91) (width 0.2) (layer "B.Cu") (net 1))
 (segment (start 136.37 45.24) (end 140.97 40.64) (width 0.2) (layer "F.Cu") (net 5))
 (segment (start 136.37 53.735) (end 135.269 52.634) (width 0.2) (layer "F.Cu") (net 5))
 (segment (start 159.9595 40.64) (end 162.125 42.8055) (width 0.2) (layer "F.Cu") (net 5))
 (segment (start 135.269 46.341) (end 136.37 45.24) (width 0.2) (layer "F.Cu") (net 5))
 (segment (start 177.8 58.4805) (end 162.125 42.8055) (width 0.2) (layer "F.Cu") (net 5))
 (segment (start 140.97 40.64) (end 159.9595 40.64) (width 0.2) (layer "F.Cu") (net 5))
 (segment (start 135.269 52.634) (end 135.269 46.341) (width 0.2) (layer "F.Cu") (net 5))
 (segment (start 177.8 59.97) (end 177.8 58.4805) (width 0.2) (layer "F.Cu") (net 5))
 (segment (start 144.78 72.39) (end 154.94 62.23) (width 0.2) (layer "F.Cu") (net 2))
 (segment (start 139.7 80.01) (end 139.7 77.47) (width 0.2) (layer "F.Cu") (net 2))
 (segment (start 154.94 62.23) (end 154.94 57.15) (width 0.2) (layer "F.Cu") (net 2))
 (segment (start 139.7 77.47) (end 142.24 74.93) (width 0.2) (layer "F.Cu") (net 2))
 (segment (start 157.8545 55.5055) (end 162.125 55.5055) (width 0.2) (layer "F.Cu") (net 2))
 (segment (start 157.48 55.88) (end 157.8545 55.5055) (width 0.2) (layer "F.Cu") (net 2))
 (via (at 144.78 72.39) (size 0.6) (drill 0.3) (layers "F.Cu" "B.Cu") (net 2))
 (via (at 154.94 57.15) (size 0.6) (drill 0.3) (layers "F.Cu" "B.Cu") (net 2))
 (via (at 157.48 55.88) (size 0.6) (drill 0.3) (layers "F.Cu" "B.Cu") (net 2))
 (via (at 142.24 74.93) (size 0.6) (drill 0.3) (layers "F.Cu" "B.Cu") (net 2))
 (segment (start 156.21 57.15) (end 157.48 55.88) (width 0.2) (layer "B.Cu") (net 2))
 (segment (start 154.94 57.15) (end 156.21 57.15) (width 0.2) (layer "B.Cu") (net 2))
 (segment (start 142.24 74.93) (end 144.78 72.39) (width 0.2) (layer "B.Cu") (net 2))
 (segment (start 129.619375 68.500625) (end 132.08 66.04) (width 0.2) (layer "F.Cu") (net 13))
 (segment (start 157.48 53.34) (end 158.75 53.34) (width 0.2) (layer "F.Cu") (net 13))
 (segment (start 135.89 63.5) (end 144.78 63.5) (width 0.2) (layer "F.Cu") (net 13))
 (segment (start 144.78 63.5) (end 154.94 53.34) (width 0.2) (layer "F.Cu") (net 13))
 (segment (start 159.1245 52.9655) (end 162.125 52.9655) (width 0.2) (layer "F.Cu") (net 13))
 (segment (start 129.619375 99.06) (end 129.619375 68.500625) (width 0.2) (layer "F.Cu") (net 13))
 (segment (start 158.75 53.34) (end 159.1245 52.9655) (width 0.2) (layer "F.Cu") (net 13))
 (via (at 132.08 66.04) (size 0.6) (drill 0.3) (layers "F.Cu" "B.Cu") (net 13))
 (via (at 135.89 63.5) (size 0.6) (drill 0.3) (layers "F.Cu" "B.Cu") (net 13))
 (via (at 157.48 53.34) (size 0.6) (drill 0.3) (layers "F.Cu" "B.Cu") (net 13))
 (via (at 154.94 53.34) (size 0.6) (drill 0.3) (layers "F.Cu" "B.Cu") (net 13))
 (segment (start 132.08 66.04) (end 134.62 63.5) (width 0.2) (layer "B.Cu") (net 13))
 (segment (start 154.94 53.34) (end 157.48 53.34) (width 0.2) (layer "B.Cu") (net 13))
 (segment (start 134.62 63.5) (end 135.89 63.5) (width 0.2) (layer "B.Cu") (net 13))
 (segment (start 157.1055 50.4255) (end 162.125 50.4255) (width 0.2) (layer "F.Cu") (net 14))
 (segment (start 156.21 49.53) (end 157.1055 50.4255) (width 0.2) (layer "F.Cu") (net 14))
 (segment (start 148.669375 99.06) (end 156.21 91.519375) (width 0.2) (layer "F.Cu") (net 14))
 (segment (start 156.21 91.519375) (end 156.21 49.53) (width 0.2) (layer "F.Cu") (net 14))
 (segment (start 182.88 59.97) (end 163.83 40.92) (width 0.2) (layer "F.Cu") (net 11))
 (segment (start 158.75 45.3455) (end 146.05 58.0455) (width 0.2) (layer "F.Cu") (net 11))
 (segment (start 163.83 40.92) (end 163.83 40.7542) (width 0.2) (layer "F.Cu") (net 11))
 (segment (start 158.75 43.18) (end 158.75 45.3455) (width 0.2) (layer "F.Cu") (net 11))
 (via (at 163.83 40.7542) (size 0.6) (drill 0.3) (layers "F.Cu" "B.Cu") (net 11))
 (via (at 158.75 43.18) (size 0.6) (drill 0.3) (layers "F.Cu" "B.Cu") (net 11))
 (segment (start 163.229 41.3552) (end 160.5748 41.3552) (width 0.2) (layer "B.Cu") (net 11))
 (segment (start 163.83 40.7542) (end 163.229 41.3552) (width 0.2) (layer "B.Cu") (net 11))
 (segment (start 160.5748 41.3552) (end 158.75 43.18) (width 0.2) (layer "B.Cu") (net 11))
 (segment (start 157.48 43.18) (end 157.48 43.2405) (width 0.2) (layer "F.Cu") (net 10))
 (segment (start 180.34 58.42) (end 162.6742 40.7542) (width 0.2) (layer "F.Cu") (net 10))
 (segment (start 162.6742 40.7542) (end 161.29 40.7542) (width 0.2) (layer "F.Cu") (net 10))
 (segment (start 157.48 43.2405) (end 145.215 55.5055) (width 0.2) (layer "F.Cu") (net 10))
 (segment (start 180.34 59.97) (end 180.34 58.42) (width 0.2) (layer "F.Cu") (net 10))
 (via (at 161.29 40.7542) (size 0.6) (drill 0.3) (layers "F.Cu" "B.Cu") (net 10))
 (via (at 157.48 43.18) (size 0.6) (drill 0.3) (layers "F.Cu" "B.Cu") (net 10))
 (segment (start 159.9058 40.7542) (end 157.48 43.18) (width 0.2) (layer "B.Cu") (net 10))
 (segment (start 161.29 40.7542) (end 159.9058 40.7542) (width 0.2) (layer "B.Cu") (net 10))
 (segment (start 134.804265 53.919265) (end 134.804265 45.904265) (width 0.2) (layer "F.Cu") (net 3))
 (segment (start 133.689265 44.420735) (end 132.87 45.24) (width 0.2) (layer "F.Cu") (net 3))
 (segment (start 134.590735 44.420735) (end 133.689265 44.420735) (width 0.2) (layer "F.Cu") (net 3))
 (segment (start 136.37 55.485) (end 134.804265 53.919265) (width 0.2) (layer "F.Cu") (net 3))
 (via (at 134.590735 44.420735) (size 0.6) (drill 0.3) (layers "F.Cu" "B.Cu") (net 3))
 (via (at 134.804265 45.904265) (size 0.6) (drill 0.3) (layers "F.Cu" "B.Cu") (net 3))
 (segment (start 134.804265 45.904265) (end 134.804265 44.634265) (width 0.2) (layer "B.Cu") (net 3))
 (segment (start 134.804265 44.634265) (end 134.590735 44.420735) (width 0.2) (layer "B.Cu") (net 3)))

